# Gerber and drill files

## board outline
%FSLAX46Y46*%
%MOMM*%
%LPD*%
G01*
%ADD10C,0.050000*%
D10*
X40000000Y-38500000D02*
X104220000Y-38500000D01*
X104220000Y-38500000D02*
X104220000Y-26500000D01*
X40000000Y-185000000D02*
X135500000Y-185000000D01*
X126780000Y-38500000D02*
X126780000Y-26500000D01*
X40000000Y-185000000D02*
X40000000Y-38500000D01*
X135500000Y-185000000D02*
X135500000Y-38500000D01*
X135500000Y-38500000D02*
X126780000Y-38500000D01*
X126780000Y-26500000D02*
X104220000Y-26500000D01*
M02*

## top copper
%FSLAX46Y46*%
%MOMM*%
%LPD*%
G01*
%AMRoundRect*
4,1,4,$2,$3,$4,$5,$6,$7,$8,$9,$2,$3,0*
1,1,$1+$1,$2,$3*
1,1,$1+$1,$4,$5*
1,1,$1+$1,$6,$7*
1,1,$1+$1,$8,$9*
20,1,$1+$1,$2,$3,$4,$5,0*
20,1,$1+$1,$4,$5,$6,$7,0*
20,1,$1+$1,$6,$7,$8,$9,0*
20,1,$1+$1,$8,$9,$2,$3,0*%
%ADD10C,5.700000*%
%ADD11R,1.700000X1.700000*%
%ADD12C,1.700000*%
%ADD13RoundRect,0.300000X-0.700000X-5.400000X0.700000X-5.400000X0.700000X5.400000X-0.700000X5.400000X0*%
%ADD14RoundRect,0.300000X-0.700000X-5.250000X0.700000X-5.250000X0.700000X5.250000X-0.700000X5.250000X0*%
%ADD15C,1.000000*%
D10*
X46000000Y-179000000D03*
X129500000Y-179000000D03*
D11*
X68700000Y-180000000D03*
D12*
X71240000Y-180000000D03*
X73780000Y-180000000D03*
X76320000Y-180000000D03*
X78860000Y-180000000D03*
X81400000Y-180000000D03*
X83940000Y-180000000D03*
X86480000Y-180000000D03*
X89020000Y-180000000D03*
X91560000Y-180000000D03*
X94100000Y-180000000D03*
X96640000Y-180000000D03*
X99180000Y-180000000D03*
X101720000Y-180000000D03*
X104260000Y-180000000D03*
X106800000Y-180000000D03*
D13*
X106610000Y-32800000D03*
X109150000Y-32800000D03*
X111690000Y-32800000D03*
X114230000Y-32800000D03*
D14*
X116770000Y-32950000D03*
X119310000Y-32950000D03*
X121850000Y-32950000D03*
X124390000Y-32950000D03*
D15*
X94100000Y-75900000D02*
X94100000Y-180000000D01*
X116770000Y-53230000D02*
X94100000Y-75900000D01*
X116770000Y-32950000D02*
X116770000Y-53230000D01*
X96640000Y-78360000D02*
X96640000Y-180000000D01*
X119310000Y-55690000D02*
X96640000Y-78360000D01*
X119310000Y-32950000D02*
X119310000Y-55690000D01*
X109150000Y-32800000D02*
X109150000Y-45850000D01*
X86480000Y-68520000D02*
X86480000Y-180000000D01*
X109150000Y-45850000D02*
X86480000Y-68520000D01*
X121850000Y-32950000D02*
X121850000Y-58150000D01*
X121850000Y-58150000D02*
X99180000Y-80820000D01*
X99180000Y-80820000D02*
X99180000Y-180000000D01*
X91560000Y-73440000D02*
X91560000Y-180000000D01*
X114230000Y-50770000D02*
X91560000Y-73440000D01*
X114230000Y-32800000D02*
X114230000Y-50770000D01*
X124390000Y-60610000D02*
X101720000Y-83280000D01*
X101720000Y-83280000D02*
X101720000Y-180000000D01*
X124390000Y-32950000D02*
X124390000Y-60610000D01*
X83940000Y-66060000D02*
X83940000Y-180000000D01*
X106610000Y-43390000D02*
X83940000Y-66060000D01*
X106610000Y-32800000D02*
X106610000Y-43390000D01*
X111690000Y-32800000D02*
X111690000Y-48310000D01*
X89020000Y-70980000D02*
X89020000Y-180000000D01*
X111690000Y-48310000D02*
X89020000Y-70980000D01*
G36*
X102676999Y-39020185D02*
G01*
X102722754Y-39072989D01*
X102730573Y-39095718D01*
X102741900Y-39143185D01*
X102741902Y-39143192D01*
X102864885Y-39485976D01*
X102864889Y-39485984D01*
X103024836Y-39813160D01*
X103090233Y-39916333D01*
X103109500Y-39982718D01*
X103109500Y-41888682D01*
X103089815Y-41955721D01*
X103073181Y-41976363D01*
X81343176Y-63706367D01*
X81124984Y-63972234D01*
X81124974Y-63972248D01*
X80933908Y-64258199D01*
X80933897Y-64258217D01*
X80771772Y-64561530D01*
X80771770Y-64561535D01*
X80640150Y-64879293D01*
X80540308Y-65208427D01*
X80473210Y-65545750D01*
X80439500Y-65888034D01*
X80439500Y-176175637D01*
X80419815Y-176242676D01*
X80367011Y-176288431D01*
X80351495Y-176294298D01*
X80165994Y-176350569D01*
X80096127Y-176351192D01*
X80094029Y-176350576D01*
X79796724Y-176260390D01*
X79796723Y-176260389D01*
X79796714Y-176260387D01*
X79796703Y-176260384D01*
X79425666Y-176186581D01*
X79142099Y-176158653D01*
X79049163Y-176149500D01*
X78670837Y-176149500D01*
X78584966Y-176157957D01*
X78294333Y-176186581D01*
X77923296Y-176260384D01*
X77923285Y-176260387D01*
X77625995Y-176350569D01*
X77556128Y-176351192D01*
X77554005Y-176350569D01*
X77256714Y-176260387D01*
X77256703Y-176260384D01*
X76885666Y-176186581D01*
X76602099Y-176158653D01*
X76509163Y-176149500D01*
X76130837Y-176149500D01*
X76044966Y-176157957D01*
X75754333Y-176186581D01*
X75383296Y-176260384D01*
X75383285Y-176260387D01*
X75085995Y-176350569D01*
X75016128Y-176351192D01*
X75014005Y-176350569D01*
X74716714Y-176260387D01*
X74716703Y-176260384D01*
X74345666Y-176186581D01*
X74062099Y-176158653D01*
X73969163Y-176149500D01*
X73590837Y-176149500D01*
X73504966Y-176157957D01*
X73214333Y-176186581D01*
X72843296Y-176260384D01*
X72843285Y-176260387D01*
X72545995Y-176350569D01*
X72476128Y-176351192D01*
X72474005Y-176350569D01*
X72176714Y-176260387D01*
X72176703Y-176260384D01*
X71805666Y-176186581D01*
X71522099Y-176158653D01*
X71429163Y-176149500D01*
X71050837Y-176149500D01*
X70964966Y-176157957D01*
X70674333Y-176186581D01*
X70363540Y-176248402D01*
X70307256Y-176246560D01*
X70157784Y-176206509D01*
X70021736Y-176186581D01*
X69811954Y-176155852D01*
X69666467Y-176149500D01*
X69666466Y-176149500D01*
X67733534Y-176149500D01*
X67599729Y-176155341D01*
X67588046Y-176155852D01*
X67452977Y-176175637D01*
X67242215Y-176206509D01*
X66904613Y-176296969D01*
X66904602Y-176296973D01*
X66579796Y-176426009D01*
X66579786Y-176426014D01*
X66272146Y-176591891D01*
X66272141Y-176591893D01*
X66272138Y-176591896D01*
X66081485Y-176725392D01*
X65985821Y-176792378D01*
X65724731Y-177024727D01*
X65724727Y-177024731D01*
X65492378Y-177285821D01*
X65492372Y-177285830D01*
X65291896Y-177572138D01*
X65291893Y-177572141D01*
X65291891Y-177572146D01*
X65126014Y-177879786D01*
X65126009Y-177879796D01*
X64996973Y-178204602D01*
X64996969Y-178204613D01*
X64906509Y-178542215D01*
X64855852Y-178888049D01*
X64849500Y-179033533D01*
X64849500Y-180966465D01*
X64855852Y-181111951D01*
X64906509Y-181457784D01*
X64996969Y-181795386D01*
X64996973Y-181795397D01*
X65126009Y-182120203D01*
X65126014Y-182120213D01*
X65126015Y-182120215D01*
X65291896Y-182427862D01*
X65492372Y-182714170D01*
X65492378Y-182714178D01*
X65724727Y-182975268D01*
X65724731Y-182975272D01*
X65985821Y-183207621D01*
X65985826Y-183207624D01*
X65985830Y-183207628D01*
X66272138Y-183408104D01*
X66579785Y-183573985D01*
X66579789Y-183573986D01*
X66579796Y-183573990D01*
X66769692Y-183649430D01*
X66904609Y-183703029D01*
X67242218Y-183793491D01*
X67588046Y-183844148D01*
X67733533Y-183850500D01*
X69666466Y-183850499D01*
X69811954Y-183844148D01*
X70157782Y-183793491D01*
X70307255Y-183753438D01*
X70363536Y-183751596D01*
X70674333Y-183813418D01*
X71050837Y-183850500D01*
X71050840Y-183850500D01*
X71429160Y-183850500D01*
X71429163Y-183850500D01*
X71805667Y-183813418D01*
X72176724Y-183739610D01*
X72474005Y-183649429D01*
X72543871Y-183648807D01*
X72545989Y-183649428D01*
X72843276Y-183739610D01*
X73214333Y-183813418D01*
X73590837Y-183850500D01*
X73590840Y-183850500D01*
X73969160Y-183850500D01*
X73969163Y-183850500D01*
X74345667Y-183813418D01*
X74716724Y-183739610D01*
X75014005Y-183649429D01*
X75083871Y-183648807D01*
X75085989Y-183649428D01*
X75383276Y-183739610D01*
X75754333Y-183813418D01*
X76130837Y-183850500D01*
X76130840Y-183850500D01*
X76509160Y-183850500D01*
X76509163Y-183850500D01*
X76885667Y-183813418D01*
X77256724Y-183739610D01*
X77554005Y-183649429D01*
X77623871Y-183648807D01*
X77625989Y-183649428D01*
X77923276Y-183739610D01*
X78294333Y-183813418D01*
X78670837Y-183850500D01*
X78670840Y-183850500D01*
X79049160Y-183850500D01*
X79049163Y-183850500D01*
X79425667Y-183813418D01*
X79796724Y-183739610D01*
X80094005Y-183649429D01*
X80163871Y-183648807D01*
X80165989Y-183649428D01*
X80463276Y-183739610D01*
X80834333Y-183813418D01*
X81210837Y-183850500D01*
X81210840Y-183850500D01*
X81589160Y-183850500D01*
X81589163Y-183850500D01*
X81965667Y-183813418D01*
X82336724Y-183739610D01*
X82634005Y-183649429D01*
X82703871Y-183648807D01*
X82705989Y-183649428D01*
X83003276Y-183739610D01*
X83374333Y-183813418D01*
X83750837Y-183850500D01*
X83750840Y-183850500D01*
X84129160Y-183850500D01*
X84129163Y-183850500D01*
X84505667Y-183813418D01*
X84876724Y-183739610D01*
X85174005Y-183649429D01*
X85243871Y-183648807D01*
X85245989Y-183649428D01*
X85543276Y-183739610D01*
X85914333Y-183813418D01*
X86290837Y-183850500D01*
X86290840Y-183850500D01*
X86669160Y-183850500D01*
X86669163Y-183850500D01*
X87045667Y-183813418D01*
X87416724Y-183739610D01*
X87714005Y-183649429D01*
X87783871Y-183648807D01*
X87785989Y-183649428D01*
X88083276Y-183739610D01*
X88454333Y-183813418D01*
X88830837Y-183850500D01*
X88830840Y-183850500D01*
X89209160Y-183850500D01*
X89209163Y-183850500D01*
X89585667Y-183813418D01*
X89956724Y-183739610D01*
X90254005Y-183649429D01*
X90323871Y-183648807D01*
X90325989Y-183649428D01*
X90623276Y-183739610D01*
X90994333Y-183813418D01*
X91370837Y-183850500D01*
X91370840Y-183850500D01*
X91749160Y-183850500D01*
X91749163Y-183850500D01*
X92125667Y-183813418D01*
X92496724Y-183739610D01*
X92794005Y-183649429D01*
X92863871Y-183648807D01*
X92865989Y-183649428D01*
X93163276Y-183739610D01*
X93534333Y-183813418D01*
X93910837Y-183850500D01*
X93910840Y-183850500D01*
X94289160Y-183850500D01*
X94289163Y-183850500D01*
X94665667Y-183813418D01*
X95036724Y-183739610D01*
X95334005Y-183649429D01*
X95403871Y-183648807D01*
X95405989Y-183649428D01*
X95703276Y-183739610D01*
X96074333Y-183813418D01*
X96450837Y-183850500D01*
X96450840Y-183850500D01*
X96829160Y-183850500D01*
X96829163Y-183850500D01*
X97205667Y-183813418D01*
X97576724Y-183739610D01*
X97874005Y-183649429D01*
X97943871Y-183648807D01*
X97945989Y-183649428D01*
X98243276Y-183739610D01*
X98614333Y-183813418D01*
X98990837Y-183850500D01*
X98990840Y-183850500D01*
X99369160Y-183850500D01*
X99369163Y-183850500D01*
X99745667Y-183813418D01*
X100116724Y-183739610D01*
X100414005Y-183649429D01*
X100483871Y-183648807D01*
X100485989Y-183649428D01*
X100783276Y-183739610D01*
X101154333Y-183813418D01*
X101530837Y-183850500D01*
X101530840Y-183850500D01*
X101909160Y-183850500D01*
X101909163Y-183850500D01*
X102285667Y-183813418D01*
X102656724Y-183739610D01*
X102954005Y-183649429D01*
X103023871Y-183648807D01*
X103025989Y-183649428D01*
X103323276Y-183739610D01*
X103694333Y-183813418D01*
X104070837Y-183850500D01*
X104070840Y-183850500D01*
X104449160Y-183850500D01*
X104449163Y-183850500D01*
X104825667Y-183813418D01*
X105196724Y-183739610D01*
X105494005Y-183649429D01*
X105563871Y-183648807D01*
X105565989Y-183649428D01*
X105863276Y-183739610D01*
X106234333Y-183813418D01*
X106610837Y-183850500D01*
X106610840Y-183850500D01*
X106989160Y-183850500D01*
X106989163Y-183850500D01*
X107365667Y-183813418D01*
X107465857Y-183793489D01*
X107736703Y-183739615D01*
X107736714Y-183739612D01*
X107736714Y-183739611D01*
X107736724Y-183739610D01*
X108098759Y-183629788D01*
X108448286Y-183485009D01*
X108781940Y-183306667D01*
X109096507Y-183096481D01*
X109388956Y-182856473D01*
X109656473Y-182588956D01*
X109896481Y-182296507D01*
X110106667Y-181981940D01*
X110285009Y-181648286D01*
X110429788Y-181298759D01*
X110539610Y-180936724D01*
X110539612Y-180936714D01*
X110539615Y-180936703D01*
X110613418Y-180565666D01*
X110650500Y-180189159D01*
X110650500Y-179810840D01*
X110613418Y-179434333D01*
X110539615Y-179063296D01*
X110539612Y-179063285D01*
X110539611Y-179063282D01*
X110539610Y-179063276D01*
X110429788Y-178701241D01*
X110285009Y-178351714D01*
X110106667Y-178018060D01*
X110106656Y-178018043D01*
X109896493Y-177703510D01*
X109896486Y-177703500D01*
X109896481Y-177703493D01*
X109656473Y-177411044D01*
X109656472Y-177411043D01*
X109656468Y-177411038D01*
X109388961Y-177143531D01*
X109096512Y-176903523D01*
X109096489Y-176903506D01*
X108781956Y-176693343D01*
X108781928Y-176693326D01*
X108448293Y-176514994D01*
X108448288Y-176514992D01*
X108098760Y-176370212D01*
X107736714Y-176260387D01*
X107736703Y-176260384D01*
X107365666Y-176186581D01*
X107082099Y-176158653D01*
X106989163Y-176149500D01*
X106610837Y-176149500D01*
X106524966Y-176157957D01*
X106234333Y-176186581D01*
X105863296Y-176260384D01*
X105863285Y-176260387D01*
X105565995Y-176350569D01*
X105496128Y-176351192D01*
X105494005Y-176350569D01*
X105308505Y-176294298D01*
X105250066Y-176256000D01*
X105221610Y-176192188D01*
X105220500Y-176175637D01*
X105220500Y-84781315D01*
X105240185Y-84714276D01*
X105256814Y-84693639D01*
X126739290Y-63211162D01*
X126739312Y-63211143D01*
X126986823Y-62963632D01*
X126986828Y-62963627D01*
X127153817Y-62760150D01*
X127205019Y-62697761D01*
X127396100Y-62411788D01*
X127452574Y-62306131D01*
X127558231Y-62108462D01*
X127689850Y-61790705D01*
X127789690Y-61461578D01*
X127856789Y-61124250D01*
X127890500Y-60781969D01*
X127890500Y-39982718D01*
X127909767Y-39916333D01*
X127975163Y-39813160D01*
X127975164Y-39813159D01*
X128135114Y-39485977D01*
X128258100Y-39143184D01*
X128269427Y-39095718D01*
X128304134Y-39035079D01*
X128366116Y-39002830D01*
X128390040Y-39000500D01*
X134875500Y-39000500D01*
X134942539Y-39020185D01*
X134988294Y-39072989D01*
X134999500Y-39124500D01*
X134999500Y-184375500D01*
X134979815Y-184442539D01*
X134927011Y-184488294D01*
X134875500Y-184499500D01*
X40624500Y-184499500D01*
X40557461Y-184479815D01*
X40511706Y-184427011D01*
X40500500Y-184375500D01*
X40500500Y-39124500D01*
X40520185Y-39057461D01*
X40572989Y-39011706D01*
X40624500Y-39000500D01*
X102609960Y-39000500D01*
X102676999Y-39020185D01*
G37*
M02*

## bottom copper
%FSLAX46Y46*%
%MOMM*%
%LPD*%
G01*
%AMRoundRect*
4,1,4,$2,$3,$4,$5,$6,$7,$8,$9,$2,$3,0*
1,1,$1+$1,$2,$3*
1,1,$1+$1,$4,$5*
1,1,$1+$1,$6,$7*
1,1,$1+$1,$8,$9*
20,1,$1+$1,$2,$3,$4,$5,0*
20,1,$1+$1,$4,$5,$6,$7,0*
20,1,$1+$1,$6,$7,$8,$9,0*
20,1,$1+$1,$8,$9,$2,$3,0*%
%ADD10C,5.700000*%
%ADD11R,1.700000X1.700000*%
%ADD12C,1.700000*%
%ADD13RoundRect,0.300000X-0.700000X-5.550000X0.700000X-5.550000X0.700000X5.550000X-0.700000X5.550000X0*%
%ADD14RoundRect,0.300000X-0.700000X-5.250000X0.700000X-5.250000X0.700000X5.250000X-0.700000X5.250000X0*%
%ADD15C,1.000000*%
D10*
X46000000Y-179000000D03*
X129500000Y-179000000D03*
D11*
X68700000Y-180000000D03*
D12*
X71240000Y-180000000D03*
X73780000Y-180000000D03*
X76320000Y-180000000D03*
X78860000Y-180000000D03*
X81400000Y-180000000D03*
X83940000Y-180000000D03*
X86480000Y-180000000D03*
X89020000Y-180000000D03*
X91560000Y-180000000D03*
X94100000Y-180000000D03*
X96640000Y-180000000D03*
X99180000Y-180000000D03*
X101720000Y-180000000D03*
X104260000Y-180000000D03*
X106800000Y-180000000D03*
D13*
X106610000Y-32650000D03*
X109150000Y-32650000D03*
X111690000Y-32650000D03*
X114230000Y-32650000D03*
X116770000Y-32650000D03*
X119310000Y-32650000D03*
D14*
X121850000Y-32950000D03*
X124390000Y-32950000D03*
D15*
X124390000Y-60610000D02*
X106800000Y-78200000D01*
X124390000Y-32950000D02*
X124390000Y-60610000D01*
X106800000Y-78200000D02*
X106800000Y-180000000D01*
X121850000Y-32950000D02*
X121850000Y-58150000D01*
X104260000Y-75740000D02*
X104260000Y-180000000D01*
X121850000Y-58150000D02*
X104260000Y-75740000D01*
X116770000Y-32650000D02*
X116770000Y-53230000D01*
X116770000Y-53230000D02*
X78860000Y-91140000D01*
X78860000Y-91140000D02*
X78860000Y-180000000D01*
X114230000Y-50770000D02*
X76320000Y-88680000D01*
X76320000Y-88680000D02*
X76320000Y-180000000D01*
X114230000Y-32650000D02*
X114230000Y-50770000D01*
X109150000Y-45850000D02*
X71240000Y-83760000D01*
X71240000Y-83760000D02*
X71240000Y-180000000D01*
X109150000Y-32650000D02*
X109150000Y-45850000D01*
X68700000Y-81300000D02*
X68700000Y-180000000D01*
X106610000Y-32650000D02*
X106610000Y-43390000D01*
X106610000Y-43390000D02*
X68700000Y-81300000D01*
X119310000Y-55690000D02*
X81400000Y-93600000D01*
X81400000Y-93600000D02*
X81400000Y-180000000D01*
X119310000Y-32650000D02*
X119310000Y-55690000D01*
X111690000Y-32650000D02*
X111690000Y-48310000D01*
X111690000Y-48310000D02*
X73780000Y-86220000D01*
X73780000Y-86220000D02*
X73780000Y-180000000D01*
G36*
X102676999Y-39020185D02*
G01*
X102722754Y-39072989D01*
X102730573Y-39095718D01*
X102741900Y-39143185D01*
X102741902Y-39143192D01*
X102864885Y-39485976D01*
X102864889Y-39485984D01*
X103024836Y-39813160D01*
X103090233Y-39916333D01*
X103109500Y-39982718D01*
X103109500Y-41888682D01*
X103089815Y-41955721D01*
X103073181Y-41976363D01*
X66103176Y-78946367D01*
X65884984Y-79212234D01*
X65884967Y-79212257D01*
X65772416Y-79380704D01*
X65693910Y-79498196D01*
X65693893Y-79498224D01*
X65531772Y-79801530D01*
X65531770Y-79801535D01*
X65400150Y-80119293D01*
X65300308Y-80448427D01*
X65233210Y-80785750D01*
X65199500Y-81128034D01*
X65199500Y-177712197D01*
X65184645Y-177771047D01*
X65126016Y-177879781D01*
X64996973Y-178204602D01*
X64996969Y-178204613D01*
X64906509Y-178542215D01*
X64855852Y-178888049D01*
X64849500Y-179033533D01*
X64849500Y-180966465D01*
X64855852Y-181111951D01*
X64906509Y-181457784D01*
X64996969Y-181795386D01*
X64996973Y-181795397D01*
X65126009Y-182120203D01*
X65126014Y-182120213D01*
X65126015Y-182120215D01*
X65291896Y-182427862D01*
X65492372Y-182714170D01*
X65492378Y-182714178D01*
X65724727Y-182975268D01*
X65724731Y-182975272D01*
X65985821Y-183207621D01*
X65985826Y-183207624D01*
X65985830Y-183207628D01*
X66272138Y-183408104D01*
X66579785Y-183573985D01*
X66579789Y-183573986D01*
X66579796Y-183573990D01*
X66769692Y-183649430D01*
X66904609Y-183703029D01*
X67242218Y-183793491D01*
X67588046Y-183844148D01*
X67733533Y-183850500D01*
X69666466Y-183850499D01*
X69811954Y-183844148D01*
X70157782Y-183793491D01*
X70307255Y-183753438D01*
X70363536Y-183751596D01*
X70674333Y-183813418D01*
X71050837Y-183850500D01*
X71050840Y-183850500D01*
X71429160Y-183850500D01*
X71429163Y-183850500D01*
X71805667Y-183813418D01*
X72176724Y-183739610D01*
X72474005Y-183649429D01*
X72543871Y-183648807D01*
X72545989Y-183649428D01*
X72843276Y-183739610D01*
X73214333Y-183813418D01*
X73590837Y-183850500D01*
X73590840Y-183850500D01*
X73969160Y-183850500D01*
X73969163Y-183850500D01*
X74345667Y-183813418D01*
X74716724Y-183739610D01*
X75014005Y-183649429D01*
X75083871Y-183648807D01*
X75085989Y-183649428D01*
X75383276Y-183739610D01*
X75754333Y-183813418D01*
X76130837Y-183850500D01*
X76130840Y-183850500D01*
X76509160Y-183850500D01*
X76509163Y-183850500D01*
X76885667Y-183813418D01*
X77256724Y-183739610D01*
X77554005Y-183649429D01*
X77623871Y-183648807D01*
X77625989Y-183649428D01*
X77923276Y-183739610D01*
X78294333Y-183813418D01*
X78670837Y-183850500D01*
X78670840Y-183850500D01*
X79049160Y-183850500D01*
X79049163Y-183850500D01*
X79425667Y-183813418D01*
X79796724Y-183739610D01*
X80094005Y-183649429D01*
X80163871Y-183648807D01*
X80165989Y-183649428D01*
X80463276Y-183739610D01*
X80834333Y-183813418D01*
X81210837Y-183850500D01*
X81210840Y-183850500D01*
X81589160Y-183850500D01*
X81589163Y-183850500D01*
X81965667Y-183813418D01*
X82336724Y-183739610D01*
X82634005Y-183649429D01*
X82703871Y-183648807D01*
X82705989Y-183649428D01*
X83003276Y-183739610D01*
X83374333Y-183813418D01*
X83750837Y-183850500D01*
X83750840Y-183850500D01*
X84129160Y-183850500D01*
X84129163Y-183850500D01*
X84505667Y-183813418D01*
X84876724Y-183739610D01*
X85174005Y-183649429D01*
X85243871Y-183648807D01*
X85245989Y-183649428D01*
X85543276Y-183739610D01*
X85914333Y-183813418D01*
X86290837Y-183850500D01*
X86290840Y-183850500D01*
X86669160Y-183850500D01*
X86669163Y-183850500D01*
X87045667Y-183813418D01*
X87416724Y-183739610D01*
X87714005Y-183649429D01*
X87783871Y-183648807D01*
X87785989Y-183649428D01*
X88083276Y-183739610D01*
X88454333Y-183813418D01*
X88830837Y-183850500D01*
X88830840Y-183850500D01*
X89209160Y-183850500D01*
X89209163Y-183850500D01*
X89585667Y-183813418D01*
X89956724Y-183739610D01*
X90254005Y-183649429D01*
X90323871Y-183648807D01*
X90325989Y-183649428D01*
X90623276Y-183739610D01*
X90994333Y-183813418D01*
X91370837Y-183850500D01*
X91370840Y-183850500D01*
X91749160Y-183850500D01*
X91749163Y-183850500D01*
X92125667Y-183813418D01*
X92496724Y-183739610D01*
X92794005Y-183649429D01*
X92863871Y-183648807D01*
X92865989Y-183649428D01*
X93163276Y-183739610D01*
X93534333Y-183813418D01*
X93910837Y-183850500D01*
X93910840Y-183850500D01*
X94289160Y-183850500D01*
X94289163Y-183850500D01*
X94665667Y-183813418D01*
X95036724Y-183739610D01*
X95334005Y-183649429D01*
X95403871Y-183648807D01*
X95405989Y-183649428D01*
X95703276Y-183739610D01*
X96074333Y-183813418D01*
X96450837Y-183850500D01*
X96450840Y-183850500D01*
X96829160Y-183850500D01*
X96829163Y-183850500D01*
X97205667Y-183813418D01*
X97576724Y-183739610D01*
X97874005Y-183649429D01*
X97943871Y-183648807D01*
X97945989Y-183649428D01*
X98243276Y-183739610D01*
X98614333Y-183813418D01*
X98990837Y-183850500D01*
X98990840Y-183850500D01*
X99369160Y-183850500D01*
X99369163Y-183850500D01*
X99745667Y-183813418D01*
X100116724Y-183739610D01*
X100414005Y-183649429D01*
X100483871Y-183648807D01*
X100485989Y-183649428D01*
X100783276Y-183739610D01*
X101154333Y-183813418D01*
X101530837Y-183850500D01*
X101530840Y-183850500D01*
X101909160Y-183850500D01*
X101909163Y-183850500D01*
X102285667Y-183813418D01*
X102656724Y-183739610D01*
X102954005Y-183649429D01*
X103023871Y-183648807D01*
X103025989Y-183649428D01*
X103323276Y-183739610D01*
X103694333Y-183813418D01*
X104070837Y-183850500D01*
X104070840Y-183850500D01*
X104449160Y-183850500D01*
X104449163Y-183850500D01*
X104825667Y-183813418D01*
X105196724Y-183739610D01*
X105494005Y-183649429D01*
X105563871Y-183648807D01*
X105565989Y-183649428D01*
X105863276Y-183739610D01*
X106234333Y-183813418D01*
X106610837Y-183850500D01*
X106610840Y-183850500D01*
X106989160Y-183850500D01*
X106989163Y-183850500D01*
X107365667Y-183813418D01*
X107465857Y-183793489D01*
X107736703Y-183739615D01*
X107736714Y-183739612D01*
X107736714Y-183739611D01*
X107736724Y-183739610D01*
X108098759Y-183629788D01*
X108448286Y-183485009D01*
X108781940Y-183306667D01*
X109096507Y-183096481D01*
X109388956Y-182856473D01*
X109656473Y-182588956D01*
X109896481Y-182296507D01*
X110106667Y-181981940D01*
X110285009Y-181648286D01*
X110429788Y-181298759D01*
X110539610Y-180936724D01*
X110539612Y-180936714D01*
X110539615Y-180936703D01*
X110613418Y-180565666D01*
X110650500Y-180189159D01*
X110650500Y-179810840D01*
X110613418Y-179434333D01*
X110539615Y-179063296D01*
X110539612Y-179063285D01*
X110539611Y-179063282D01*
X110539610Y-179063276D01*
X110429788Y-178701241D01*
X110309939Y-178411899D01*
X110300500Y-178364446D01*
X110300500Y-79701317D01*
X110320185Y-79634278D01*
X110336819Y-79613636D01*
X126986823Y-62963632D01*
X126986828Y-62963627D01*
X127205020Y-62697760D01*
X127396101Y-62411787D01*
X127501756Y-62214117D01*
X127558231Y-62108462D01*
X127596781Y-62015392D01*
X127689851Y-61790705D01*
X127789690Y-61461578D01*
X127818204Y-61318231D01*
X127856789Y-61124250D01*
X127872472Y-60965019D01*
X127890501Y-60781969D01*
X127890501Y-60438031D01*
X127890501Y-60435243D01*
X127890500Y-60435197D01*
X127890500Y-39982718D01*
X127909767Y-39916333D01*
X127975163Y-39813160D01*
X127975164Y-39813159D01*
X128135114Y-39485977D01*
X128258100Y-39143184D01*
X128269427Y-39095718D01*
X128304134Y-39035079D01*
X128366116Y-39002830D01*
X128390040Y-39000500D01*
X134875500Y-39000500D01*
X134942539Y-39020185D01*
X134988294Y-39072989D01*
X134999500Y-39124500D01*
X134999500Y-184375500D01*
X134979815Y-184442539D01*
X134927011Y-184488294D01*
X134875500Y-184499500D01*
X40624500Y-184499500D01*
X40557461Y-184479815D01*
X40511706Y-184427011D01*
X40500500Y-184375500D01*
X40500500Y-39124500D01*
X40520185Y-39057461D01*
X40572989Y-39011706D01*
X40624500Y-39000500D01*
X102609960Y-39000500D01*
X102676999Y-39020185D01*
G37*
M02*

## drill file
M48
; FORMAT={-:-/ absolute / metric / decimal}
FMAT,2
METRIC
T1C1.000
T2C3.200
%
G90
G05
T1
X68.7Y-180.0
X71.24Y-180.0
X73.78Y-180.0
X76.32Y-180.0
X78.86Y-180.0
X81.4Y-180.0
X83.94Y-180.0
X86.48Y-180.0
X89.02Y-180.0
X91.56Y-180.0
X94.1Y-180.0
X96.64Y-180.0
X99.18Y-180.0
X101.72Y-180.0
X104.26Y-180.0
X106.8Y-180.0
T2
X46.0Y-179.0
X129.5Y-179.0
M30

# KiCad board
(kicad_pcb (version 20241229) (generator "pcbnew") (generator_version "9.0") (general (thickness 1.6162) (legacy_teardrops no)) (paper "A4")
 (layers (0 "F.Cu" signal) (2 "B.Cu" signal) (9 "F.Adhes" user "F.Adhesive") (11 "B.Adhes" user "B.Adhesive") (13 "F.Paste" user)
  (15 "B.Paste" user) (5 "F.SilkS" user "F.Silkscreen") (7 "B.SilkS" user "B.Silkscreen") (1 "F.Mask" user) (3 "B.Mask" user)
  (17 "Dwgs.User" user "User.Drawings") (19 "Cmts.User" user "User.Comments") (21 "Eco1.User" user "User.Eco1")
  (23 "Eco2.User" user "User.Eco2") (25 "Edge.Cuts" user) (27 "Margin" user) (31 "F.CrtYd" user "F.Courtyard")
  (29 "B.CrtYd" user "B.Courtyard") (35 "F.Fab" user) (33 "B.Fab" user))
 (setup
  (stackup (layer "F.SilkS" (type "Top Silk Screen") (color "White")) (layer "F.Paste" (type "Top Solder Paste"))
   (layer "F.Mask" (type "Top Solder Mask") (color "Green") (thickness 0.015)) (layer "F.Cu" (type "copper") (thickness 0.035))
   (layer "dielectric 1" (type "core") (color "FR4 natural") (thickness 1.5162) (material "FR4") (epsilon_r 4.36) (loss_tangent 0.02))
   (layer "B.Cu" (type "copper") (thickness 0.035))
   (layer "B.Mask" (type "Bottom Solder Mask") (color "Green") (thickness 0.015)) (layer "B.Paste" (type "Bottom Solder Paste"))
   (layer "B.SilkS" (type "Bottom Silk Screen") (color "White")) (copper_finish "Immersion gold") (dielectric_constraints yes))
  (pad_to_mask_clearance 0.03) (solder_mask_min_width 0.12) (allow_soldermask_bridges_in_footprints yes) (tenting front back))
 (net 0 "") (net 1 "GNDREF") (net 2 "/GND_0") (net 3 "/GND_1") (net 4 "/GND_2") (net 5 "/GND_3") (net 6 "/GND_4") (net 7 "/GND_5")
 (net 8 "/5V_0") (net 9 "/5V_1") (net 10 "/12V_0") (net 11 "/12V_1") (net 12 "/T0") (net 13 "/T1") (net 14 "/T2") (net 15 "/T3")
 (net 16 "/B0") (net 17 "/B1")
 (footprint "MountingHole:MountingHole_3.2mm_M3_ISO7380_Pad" (layer "F.Cu") (at 46 179)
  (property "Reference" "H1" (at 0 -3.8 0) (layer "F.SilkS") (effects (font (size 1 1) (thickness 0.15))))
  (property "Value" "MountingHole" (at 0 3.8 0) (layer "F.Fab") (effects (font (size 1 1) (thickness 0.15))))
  (pad "1" thru_hole circle (at 0 0) (size 5.7 5.7) (drill 3.2) (layers "*.Cu" "*.Mask") (remove_unused_layers no) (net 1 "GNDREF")
   (zone_connect 2)))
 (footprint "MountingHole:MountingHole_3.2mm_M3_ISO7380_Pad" (layer "F.Cu") (at 129.5 179)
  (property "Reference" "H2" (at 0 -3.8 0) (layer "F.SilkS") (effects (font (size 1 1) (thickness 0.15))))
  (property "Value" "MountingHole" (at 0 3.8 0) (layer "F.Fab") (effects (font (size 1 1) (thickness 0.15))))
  (pad "1" thru_hole circle (at 0 0) (size 5.7 5.7) (drill 3.2) (layers "*.Cu" "*.Mask") (remove_unused_layers no) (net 1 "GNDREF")
   (zone_connect 2)))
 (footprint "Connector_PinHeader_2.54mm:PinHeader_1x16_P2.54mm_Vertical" (layer "F.Cu") (at 68.7 180 90)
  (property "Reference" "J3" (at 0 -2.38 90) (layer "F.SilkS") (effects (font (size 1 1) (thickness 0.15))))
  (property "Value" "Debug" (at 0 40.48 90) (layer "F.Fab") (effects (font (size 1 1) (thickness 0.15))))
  (pad "1" thru_hole rect (at 0 0 90) (size 1.7 1.7) (drill 1) (layers "*.Cu" "*.Mask") (remove_unused_layers no) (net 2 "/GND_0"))
  (pad "2" thru_hole circle (at 0 2.54 90) (size 1.7 1.7) (drill 1) (layers "*.Cu" "*.Mask") (remove_unused_layers no) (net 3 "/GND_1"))
  (pad "3" thru_hole circle (at 0 5.08 90) (size 1.7 1.7) (drill 1) (layers "*.Cu" "*.Mask") (remove_unused_layers no) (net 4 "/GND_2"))
  (pad "4" thru_hole circle (at 0 7.62 90) (size 1.7 1.7) (drill 1) (layers "*.Cu" "*.Mask") (remove_unused_layers no) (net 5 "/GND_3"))
  (pad "5" thru_hole circle (at 0 10.16 90) (size 1.7 1.7) (drill 1) (layers "*.Cu" "*.Mask") (remove_unused_layers no) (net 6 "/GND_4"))
  (pad "6" thru_hole circle (at 0 12.7 90) (size 1.7 1.7) (drill 1) (layers "*.Cu" "*.Mask") (remove_unused_layers no) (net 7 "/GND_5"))
  (pad "7" thru_hole circle (at 0 15.24 90) (size 1.7 1.7) (drill 1) (layers "*.Cu" "*.Mask") (remove_unused_layers no) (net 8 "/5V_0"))
  (pad "8" thru_hole circle (at 0 17.78 90) (size 1.7 1.7) (drill 1) (layers "*.Cu" "*.Mask") (remove_unused_layers no) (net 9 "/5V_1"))
  (pad "9" thru_hole circle (at 0 20.32 90) (size 1.7 1.7) (drill 1) (layers "*.Cu" "*.Mask") (remove_unused_layers no) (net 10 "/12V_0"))
  (pad "10" thru_hole circle (at 0 22.86 90) (size 1.7 1.7) (drill 1) (layers "*.Cu" "*.Mask") (remove_unused_layers no) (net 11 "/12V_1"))
  (pad "11" thru_hole circle (at 0 25.4 90) (size 1.7 1.7) (drill 1) (layers "*.Cu" "*.Mask") (remove_unused_layers no) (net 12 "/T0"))
  (pad "12" thru_hole circle (at 0 27.94 90) (size 1.7 1.7) (drill 1) (layers "*.Cu" "*.Mask") (remove_unused_layers no) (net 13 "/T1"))
  (pad "13" thru_hole circle (at 0 30.48 90) (size 1.7 1.7) (drill 1) (layers "*.Cu" "*.Mask") (remove_unused_layers no) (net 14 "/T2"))
  (pad "14" thru_hole circle (at 0 33.02 90) (size 1.7 1.7) (drill 1) (layers "*.Cu" "*.Mask") (remove_unused_layers no) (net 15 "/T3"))
  (pad "15" thru_hole circle (at 0 35.56 90) (size 1.7 1.7) (drill 1) (layers "*.Cu" "*.Mask") (remove_unused_layers no) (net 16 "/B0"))
  (pad "16" thru_hole circle (at 0 38.1 90) (size 1.7 1.7) (drill 1) (layers "*.Cu" "*.Mask") (remove_unused_layers no) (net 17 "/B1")))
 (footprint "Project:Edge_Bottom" (layer "F.Cu") (at 115.5 38.5)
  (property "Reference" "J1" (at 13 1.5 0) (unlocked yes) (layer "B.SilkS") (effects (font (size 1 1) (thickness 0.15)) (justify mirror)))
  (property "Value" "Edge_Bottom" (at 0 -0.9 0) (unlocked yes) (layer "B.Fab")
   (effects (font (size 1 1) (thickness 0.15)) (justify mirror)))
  (pad "1" smd roundrect (at -8.89 -5.85) (size 2 11.7) (layers "B.Cu" "B.Mask" "B.Paste") (roundrect_rratio 0.15) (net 2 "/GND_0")
   (thermal_bridge_angle 45))
  (pad "2" smd roundrect (at -6.35 -5.85) (size 2 11.7) (layers "B.Cu" "B.Mask" "B.Paste") (roundrect_rratio 0.15) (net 3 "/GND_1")
   (thermal_bridge_angle 45))
  (pad "3" smd roundrect (at -3.81 -5.85) (size 2 11.7) (layers "B.Cu" "B.Mask" "B.Paste") (roundrect_rratio 0.15) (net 4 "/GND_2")
   (thermal_bridge_angle 45))
  (pad "4" smd roundrect (at -1.27 -5.85) (size 2 11.7) (layers "B.Cu" "B.Mask" "B.Paste") (roundrect_rratio 0.15) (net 5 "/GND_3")
   (thermal_bridge_angle 45))
  (pad "5" smd roundrect (at 1.27 -5.85) (size 2 11.7) (layers "B.Cu" "B.Mask" "B.Paste") (roundrect_rratio 0.15) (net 6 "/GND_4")
   (thermal_bridge_angle 45))
  (pad "6" smd roundrect (at 3.81 -5.85) (size 2 11.7) (layers "B.Cu" "B.Mask" "B.Paste") (roundrect_rratio 0.15) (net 7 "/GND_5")
   (thermal_bridge_angle 45))
  (pad "7" smd roundrect (at 6.35 -5.55) (size 2 11.1) (layers "B.Cu" "B.Mask" "B.Paste") (roundrect_rratio 0.15) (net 16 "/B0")
   (thermal_bridge_angle 45))
  (pad "8" smd roundrect (at 8.89 -5.55) (size 2 11.1) (layers "B.Cu" "B.Mask" "B.Paste") (roundrect_rratio 0.15) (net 17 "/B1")
   (thermal_bridge_angle 45)))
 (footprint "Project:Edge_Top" (layer "F.Cu") (at 115.5 38.5)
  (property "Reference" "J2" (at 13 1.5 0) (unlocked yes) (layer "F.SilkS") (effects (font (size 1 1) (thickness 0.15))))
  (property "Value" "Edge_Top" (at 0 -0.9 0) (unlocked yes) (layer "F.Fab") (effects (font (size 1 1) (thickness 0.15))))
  (pad "1" smd roundrect (at -8.89 -5.7) (size 2 11.4) (layers "F.Cu" "F.Mask" "F.Paste") (roundrect_rratio 0.15) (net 8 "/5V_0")
   (thermal_bridge_angle 45))
  (pad "2" smd roundrect (at -6.35 -5.7) (size 2 11.4) (layers "F.Cu" "F.Mask" "F.Paste") (roundrect_rratio 0.15) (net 9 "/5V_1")
   (thermal_bridge_angle 45))
  (pad "3" smd roundrect (at -3.81 -5.7) (size 2 11.4) (layers "F.Cu" "F.Mask" "F.Paste") (roundrect_rratio 0.15) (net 10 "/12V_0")
   (thermal_bridge_angle 45))
  (pad "4" smd roundrect (at -1.27 -5.7) (size 2 11.4) (layers "F.Cu" "F.Mask" "F.Paste") (roundrect_rratio 0.15) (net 11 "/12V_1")
   (thermal_bridge_angle 45))
  (pad "5" smd roundrect (at 1.27 -5.55) (size 2 11.1) (layers "F.Cu" "F.Mask" "F.Paste") (roundrect_rratio 0.15) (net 12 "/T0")
   (thermal_bridge_angle 45))
  (pad "6" smd roundrect (at 3.81 -5.55) (size 2 11.1) (layers "F.Cu" "F.Mask" "F.Paste") (roundrect_rratio 0.15) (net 13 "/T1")
   (thermal_bridge_angle 45))
  (pad "7" smd roundrect (at 6.35 -5.55) (size 2 11.1) (layers "F.Cu" "F.Mask" "F.Paste") (roundrect_rratio 0.15) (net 14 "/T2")
   (thermal_bridge_angle 45))
  (pad "8" smd roundrect (at 8.89 -5.55) (size 2 11.1) (layers "F.Cu" "F.Mask" "F.Paste") (roundrect_rratio 0.15) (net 15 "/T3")
   (thermal_bridge_angle 45)))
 (gr_line (start 40 38.5) (end 104.22 38.5) (stroke (width 0.05) (type default)) (layer "Edge.Cuts"))
 (gr_line (start 104.22 38.5) (end 104.22 26.5) (stroke (width 0.05) (type default)) (layer "Edge.Cuts"))
 (gr_line (start 40 185) (end 135.5 185) (stroke (width 0.05) (type default)) (layer "Edge.Cuts"))
 (gr_line (start 126.78 38.5) (end 126.78 26.5) (stroke (width 0.05) (type default)) (layer "Edge.Cuts"))
 (gr_line (start 40 185) (end 40 38.5) (stroke (width 0.05) (type default)) (layer "Edge.Cuts"))
 (gr_line (start 135.5 185) (end 135.5 38.5) (stroke (width 0.05) (type default)) (layer "Edge.Cuts"))
 (gr_line (start 135.5 38.5) (end 126.78 38.5) (stroke (width 0.05) (type default)) (layer "Edge.Cuts"))
 (gr_line (start 126.78 26.5) (end 104.22 26.5) (stroke (width 0.05) (type default)) (layer "Edge.Cuts"))
 (segment (start 124.39 60.61) (end 106.8 78.2) (width 1) (layer "B.Cu") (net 17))
 (segment (start 124.39 32.95) (end 124.39 60.61) (width 1) (layer "B.Cu") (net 17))
 (segment (start 106.8 78.2) (end 106.8 180) (width 1) (layer "B.Cu") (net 17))
 (segment (start 121.85 32.95) (end 121.85 58.15) (width 1) (layer "B.Cu") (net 16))
 (segment (start 104.26 75.74) (end 104.26 180) (width 1) (layer "B.Cu") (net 16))
 (segment (start 121.85 58.15) (end 104.26 75.74) (width 1) (layer "B.Cu") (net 16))
 (segment (start 116.77 32.65) (end 116.77 53.23) (width 1) (layer "B.Cu") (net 6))
 (segment (start 116.77 53.23) (end 78.86 91.14) (width 1) (layer "B.Cu") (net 6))
 (segment (start 78.86 91.14) (end 78.86 180) (width 1) (layer "B.Cu") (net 6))
 (segment (start 114.23 50.77) (end 76.32 88.68) (width 1) (layer "B.Cu") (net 5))
 (segment (start 76.32 88.68) (end 76.32 180) (width 1) (layer "B.Cu") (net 5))
 (segment (start 114.23 32.65) (end 114.23 50.77) (width 1) (layer "B.Cu") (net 5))
 (segment (start 109.15 45.85) (end 71.24 83.76) (width 1) (layer "B.Cu") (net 3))
 (segment (start 71.24 83.76) (end 71.24 180) (width 1) (layer "B.Cu") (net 3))
 (segment (start 109.15 32.65) (end 109.15 45.85) (width 1) (layer "B.Cu") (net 3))
 (segment (start 68.7 81.3) (end 68.7 180) (width 1) (layer "B.Cu") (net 2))
 (segment (start 106.61 32.65) (end 106.61 43.39) (width 1) (layer "B.Cu") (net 2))
 (segment (start 106.61 43.39) (end 68.7 81.3) (width 1) (layer "B.Cu") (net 2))
 (segment (start 119.31 55.69) (end 81.4 93.6) (width 1) (layer "B.Cu") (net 7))
 (segment (start 81.4 93.6) (end 81.4 180) (width 1) (layer "B.Cu") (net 7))
 (segment (start 119.31 32.65) (end 119.31 55.69) (width 1) (layer "B.Cu") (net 7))
 (segment (start 111.69 32.65) (end 111.69 48.31) (width 1) (layer "B.Cu") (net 4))
 (segment (start 111.69 48.31) (end 73.78 86.22) (width 1) (layer "B.Cu") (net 4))
 (segment (start 73.78 86.22) (end 73.78 180) (width 1) (layer "B.Cu") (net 4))
 (segment (start 94.1 75.9) (end 94.1 180) (width 1) (layer "F.Cu") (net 12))
 (segment (start 116.77 53.23) (end 94.1 75.9) (width 1) (layer "F.Cu") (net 12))
 (segment (start 116.77 32.95) (end 116.77 53.23) (width 1) (layer "F.Cu") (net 12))
 (segment (start 96.64 78.36) (end 96.64 180) (width 1) (layer "F.Cu") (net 13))
 (segment (start 119.31 55.69) (end 96.64 78.36) (width 1) (layer "F.Cu") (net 13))
 (segment (start 119.31 32.95) (end 119.31 55.69) (width 1) (layer "F.Cu") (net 13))
 (segment (start 109.15 32.8) (end 109.15 45.85) (width 1) (layer "F.Cu") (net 9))
 (segment (start 86.48 68.52) (end 86.48 180) (width 1) (layer "F.Cu") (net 9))
 (segment (start 109.15 45.85) (end 86.48 68.52) (width 1) (layer "F.Cu") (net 9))
 (segment (start 121.85 32.95) (end 121.85 58.15) (width 1) (layer "F.Cu") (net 14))
 (segment (start 121.85 58.15) (end 99.18 80.82) (width 1) (layer "F.Cu") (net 14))
 (segment (start 99.18 80.82) (end 99.18 180) (width 1) (layer "F.Cu") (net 14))
 (segment (start 91.56 73.44) (end 91.56 180) (width 1) (layer "F.Cu") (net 11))
 (segment (start 114.23 50.77) (end 91.56 73.44) (width 1) (layer "F.Cu") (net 11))
 (segment (start 114.23 32.8) (end 114.23 50.77) (width 1) (layer "F.Cu") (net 11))
 (segment (start 124.39 60.61) (end 101.72 83.28) (width 1) (layer "F.Cu") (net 15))
 (segment (start 101.72 83.28) (end 101.72 180) (width 1) (layer "F.Cu") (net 15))
 (segment (start 124.39 32.95) (end 124.39 60.61) (width 1) (layer "F.Cu") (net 15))
 (segment (start 83.94 66.06) (end 83.94 180) (width 1) (layer "F.Cu") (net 8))
 (segment (start 106.61 43.39) (end 83.94 66.06) (width 1) (layer "F.Cu") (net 8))
 (segment (start 106.61 32.8) (end 106.61 43.39) (width 1) (layer "F.Cu") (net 8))
 (segment (start 111.69 32.8) (end 111.69 48.31) (width 1) (layer "F.Cu") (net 10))
 (segment (start 89.02 70.98) (end 89.02 180) (width 1) (layer "F.Cu") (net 10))
 (segment (start 111.69 48.31) (end 89.02 70.98) (width 1) (layer "F.Cu") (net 10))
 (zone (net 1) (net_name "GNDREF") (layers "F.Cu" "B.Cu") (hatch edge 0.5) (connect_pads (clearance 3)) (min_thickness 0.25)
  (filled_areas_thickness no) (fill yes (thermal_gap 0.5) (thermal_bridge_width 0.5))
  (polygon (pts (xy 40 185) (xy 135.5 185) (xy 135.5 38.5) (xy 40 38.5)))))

